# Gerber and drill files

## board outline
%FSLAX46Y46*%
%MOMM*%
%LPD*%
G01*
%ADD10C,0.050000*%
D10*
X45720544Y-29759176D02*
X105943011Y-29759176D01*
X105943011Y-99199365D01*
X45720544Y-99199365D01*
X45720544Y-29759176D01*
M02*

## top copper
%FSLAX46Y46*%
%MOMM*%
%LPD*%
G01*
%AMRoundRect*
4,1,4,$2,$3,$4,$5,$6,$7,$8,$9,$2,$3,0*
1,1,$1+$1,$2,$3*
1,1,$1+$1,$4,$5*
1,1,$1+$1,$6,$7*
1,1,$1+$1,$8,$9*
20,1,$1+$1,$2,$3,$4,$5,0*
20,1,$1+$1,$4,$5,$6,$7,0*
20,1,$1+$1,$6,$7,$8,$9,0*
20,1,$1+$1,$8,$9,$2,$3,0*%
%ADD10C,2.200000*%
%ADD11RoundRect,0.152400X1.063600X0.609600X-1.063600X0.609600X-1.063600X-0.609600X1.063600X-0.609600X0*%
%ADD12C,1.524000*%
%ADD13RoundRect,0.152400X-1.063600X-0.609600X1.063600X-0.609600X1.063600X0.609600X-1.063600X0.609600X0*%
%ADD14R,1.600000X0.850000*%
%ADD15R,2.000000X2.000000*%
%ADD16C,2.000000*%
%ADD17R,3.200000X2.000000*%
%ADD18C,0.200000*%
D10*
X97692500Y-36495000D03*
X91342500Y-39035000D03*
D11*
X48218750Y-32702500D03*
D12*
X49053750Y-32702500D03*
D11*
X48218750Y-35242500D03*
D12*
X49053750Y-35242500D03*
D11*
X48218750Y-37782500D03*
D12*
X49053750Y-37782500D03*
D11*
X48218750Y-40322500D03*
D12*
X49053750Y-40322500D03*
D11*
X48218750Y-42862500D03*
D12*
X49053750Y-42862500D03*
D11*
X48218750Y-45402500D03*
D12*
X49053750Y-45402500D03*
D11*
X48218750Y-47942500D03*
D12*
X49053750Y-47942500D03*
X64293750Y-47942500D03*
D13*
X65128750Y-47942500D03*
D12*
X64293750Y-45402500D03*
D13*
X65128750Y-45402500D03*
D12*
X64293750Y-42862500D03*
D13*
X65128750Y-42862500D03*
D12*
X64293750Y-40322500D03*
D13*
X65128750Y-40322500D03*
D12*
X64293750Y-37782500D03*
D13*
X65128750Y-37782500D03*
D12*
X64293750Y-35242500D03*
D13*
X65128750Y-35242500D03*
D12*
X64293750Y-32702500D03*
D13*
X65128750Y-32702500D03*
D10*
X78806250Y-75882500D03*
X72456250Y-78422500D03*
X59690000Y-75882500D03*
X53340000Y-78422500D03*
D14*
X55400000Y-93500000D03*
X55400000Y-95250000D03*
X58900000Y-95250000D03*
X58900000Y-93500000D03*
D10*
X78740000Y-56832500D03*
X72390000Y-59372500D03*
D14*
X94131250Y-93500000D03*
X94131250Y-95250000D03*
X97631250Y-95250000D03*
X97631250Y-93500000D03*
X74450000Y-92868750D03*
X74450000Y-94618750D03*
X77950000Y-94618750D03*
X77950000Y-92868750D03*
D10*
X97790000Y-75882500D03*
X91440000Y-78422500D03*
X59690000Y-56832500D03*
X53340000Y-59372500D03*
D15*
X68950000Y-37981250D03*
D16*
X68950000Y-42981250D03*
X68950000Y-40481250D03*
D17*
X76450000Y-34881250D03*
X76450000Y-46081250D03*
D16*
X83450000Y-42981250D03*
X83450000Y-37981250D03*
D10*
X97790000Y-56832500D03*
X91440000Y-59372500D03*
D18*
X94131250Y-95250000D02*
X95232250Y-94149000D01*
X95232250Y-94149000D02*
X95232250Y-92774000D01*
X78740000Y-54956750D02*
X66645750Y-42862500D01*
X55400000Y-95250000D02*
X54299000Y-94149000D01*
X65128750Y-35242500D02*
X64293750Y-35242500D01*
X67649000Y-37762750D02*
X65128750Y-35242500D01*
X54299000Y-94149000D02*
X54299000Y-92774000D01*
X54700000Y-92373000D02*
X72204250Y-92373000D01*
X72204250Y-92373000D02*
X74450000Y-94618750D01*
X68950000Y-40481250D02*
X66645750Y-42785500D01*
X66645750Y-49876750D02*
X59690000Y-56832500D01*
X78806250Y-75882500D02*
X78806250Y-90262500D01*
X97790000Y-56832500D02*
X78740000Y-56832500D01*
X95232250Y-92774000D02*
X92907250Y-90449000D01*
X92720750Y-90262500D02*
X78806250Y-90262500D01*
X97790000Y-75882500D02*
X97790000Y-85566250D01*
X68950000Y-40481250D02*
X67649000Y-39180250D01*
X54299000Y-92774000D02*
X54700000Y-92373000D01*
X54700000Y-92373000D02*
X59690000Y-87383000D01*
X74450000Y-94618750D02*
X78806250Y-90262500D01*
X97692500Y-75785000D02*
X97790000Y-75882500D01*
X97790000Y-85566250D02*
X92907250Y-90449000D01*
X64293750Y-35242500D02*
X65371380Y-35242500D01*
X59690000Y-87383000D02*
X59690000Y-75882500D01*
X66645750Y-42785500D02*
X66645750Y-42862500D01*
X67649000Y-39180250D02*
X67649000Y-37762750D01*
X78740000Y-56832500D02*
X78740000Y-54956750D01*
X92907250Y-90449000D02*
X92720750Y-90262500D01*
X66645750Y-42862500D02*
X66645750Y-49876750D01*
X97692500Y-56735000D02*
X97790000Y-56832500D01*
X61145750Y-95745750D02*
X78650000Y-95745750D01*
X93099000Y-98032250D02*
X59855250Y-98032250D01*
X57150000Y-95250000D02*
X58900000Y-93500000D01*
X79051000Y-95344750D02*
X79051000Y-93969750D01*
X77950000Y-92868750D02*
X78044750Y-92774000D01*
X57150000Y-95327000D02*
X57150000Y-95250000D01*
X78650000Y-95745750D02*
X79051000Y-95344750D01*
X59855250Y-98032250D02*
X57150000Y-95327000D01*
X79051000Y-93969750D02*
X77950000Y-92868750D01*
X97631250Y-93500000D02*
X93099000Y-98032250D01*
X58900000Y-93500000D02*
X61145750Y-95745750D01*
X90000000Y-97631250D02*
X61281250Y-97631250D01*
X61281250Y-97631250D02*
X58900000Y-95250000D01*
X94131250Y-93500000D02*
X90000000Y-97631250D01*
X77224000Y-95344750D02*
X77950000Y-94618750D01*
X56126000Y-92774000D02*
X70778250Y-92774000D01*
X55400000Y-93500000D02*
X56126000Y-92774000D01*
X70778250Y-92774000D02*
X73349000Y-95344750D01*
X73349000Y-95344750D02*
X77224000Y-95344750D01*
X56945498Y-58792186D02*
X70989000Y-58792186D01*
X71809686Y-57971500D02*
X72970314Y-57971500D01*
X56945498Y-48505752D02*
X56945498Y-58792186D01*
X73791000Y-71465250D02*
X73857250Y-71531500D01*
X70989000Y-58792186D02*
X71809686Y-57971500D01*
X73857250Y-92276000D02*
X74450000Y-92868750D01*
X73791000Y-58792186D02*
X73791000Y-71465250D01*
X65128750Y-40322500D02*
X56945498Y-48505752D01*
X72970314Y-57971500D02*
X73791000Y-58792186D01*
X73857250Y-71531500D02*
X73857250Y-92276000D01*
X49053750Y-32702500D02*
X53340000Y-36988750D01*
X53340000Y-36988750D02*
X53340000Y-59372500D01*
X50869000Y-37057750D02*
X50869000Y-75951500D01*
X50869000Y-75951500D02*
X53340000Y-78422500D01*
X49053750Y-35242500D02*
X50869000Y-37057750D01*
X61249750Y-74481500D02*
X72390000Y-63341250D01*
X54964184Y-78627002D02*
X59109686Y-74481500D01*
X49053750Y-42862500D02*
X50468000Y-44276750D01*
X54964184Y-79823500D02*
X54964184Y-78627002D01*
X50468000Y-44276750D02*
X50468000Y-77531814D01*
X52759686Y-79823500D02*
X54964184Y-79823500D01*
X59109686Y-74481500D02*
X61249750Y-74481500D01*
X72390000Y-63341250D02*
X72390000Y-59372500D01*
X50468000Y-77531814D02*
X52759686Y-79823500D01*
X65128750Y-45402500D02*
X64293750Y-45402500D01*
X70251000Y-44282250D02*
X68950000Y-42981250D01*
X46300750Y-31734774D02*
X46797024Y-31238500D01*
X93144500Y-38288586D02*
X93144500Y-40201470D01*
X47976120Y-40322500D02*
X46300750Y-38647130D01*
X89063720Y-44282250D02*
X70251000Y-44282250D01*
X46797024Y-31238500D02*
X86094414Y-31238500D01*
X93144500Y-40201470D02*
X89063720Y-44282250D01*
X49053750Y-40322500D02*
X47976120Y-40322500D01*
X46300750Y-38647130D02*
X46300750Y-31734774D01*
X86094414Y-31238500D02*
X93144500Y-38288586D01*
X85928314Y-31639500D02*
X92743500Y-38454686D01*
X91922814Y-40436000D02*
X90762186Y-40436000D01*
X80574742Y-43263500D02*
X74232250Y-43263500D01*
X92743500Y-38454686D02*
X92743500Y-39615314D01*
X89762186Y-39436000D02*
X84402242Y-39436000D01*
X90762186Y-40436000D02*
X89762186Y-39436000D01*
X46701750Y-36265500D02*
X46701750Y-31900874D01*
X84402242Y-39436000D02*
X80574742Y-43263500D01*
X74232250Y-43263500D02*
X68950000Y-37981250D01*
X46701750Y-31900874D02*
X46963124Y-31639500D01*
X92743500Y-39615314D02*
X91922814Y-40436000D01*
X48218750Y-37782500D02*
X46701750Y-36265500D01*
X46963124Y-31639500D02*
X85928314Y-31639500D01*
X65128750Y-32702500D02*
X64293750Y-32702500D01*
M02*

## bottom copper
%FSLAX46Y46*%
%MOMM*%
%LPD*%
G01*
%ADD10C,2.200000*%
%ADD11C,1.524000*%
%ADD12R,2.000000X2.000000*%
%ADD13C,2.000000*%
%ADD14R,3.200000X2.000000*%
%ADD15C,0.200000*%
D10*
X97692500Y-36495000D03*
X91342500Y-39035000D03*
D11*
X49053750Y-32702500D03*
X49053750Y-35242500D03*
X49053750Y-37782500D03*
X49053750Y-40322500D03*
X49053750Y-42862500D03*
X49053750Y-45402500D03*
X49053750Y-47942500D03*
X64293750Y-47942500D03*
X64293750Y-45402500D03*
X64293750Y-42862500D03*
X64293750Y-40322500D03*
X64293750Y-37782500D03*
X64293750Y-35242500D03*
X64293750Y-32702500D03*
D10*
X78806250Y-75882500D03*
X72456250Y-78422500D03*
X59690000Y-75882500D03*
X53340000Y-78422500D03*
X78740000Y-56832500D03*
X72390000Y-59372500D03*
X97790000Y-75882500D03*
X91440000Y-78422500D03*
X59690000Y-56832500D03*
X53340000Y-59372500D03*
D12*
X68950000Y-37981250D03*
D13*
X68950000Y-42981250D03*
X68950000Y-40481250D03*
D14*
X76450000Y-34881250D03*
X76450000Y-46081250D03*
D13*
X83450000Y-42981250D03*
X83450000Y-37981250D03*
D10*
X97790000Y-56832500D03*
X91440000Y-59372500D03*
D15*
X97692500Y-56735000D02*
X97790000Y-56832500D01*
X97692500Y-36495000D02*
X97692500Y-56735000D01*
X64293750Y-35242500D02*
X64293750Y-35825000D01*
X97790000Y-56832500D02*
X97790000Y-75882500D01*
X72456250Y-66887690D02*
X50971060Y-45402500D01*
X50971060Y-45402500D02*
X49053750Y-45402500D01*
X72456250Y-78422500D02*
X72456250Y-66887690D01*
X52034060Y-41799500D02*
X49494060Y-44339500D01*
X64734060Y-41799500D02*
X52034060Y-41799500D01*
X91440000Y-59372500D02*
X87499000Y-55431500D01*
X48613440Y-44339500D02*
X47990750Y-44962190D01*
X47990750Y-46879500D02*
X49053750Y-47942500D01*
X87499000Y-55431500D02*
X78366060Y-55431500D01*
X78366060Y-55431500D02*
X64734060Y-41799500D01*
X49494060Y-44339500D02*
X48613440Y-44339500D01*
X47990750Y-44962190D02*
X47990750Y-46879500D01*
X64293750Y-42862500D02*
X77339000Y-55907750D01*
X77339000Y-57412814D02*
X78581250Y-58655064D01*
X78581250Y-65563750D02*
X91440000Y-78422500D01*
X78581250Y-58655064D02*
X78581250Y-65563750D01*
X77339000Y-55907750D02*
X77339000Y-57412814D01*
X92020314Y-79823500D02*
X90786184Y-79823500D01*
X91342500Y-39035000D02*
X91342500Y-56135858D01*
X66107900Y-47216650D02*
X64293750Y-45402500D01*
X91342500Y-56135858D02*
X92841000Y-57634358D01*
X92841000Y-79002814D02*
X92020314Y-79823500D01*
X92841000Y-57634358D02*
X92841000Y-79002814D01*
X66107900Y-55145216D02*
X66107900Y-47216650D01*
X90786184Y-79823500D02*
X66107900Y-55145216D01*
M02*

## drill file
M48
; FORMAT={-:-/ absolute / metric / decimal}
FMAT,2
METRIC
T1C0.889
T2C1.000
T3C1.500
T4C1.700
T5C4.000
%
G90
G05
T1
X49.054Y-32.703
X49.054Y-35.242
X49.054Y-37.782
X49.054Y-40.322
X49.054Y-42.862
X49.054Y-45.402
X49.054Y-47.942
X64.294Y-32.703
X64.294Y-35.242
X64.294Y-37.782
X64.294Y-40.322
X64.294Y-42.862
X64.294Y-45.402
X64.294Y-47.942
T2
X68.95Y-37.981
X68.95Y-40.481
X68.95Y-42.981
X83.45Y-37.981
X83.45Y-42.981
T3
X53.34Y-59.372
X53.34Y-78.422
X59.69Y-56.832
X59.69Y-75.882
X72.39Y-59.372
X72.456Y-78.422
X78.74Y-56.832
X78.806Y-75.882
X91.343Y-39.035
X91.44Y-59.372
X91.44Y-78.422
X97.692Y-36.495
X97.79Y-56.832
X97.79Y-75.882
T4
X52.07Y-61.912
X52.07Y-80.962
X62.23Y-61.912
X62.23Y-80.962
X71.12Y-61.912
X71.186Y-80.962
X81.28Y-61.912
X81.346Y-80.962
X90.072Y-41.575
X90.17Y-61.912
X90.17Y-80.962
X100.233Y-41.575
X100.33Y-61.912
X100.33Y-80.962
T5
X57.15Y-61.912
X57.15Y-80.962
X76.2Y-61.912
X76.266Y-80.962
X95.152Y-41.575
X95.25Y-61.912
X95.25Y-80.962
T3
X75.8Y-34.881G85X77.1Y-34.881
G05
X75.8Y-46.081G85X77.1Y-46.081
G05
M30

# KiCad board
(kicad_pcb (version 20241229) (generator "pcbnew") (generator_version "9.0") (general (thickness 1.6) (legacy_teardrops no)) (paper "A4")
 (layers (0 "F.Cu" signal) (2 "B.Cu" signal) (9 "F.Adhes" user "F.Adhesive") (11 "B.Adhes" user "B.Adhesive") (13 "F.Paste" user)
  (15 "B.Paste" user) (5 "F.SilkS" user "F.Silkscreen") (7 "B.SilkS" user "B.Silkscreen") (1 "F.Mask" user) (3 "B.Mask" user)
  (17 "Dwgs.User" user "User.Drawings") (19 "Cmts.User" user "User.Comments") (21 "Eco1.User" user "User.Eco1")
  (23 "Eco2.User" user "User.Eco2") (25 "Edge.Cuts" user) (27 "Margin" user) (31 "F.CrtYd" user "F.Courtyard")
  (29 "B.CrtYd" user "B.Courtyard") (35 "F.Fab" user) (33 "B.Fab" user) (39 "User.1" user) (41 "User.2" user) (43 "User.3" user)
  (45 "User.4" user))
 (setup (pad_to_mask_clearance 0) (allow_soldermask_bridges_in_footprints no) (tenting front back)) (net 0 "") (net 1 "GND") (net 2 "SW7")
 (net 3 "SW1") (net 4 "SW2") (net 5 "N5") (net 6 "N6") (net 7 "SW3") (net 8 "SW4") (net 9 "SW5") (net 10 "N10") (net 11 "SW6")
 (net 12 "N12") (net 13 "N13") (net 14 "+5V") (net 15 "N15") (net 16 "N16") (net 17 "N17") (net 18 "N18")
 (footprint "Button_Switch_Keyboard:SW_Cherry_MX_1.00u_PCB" (layer "F.Cu") (at 97.6925 36.495)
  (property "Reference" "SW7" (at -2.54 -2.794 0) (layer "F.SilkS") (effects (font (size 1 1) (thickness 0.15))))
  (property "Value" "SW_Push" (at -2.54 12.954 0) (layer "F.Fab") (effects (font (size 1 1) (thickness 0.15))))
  (pad "" np_thru_hole circle (at -7.62 5.08) (size 1.7 1.7) (drill 1.7) (layers "*.Cu" "*.Mask"))
  (pad "" np_thru_hole circle (at -2.54 5.08) (size 4 4) (drill 4) (layers "*.Cu" "*.Mask"))
  (pad "" np_thru_hole circle (at 2.54 5.08) (size 1.7 1.7) (drill 1.7) (layers "*.Cu" "*.Mask"))
  (pad "1" thru_hole circle (at 0 0) (size 2.2 2.2) (drill 1.5) (layers "*.Cu" "*.Mask") (remove_unused_layers no) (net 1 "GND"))
  (pad "2" thru_hole circle (at -6.35 2.54) (size 2.2 2.2) (drill 1.5) (layers "*.Cu" "*.Mask") (remove_unused_layers no) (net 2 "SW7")))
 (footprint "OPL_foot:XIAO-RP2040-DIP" (layer "F.Cu") (at 56.67375 40.3225)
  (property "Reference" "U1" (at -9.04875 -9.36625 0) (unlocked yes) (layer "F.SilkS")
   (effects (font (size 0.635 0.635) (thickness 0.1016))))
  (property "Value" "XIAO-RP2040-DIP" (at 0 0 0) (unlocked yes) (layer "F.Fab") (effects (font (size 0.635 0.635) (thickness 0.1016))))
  (pad "1" smd roundrect (at -8.455 -7.62 180) (size 2.432 1.524) (layers "F.Cu" "F.Mask") (roundrect_rratio 0.1) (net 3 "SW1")
   (thermal_bridge_angle 45))
  (pad "1" thru_hole circle (at -7.62 -7.62 180) (size 1.524 1.524) (drill 0.889) (layers "*.Cu" "*.Mask") (remove_unused_layers no)
   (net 3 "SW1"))
  (pad "2" smd roundrect (at -8.455 -5.08 180) (size 2.432 1.524) (layers "F.Cu" "F.Mask") (roundrect_rratio 0.1) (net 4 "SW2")
   (thermal_bridge_angle 45))
  (pad "2" thru_hole circle (at -7.62 -5.08 180) (size 1.524 1.524) (drill 0.889) (layers "*.Cu" "*.Mask") (remove_unused_layers no)
   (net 4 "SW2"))
  (pad "3" smd roundrect (at -8.455 -2.54 180) (size 2.432 1.524) (layers "F.Cu" "F.Mask") (roundrect_rratio 0.1) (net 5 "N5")
   (thermal_bridge_angle 45))
  (pad "3" thru_hole circle (at -7.62 -2.54 180) (size 1.524 1.524) (drill 0.889) (layers "*.Cu" "*.Mask") (remove_unused_layers no)
   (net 5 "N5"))
  (pad "4" smd roundrect (at -8.455 0 180) (size 2.432 1.524) (layers "F.Cu" "F.Mask") (roundrect_rratio 0.1) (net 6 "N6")
   (thermal_bridge_angle 45))
  (pad "4" thru_hole circle (at -7.62 0 180) (size 1.524 1.524) (drill 0.889) (layers "*.Cu" "*.Mask") (remove_unused_layers no)
   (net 6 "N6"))
  (pad "5" smd roundrect (at -8.455 2.54 180) (size 2.432 1.524) (layers "F.Cu" "F.Mask") (roundrect_rratio 0.1) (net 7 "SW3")
   (thermal_bridge_angle 45))
  (pad "5" thru_hole circle (at -7.62 2.54 180) (size 1.524 1.524) (drill 0.889) (layers "*.Cu" "*.Mask") (remove_unused_layers no)
   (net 7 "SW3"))
  (pad "6" smd roundrect (at -8.455 5.08 180) (size 2.432 1.524) (layers "F.Cu" "F.Mask") (roundrect_rratio 0.1) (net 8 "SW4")
   (thermal_bridge_angle 45))
  (pad "6" thru_hole circle (at -7.62 5.08 180) (size 1.524 1.524) (drill 0.889) (layers "*.Cu" "*.Mask") (remove_unused_layers no)
   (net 8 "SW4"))
  (pad "7" smd roundrect (at -8.455 7.62 180) (size 2.432 1.524) (layers "F.Cu" "F.Mask") (roundrect_rratio 0.1) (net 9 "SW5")
   (thermal_bridge_angle 45))
  (pad "7" thru_hole circle (at -7.62 7.62 180) (size 1.524 1.524) (drill 0.889) (layers "*.Cu" "*.Mask") (remove_unused_layers no)
   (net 9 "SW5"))
  (pad "8" thru_hole circle (at 7.62 7.62) (size 1.524 1.524) (drill 0.889) (layers "*.Cu" "*.Mask") (remove_unused_layers no)
   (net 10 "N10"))
  (pad "8" smd roundrect (at 8.455 7.62) (size 2.432 1.524) (layers "F.Cu" "F.Mask") (roundrect_rratio 0.1) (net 10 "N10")
   (thermal_bridge_angle 45))
  (pad "9" thru_hole circle (at 7.62 5.08) (size 1.524 1.524) (drill 0.889) (layers "*.Cu" "*.Mask") (remove_unused_layers no) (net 2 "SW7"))
  (pad "9" smd roundrect (at 8.455 5.08) (size 2.432 1.524) (layers "F.Cu" "F.Mask") (roundrect_rratio 0.1) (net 2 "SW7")
   (thermal_bridge_angle 45))
  (pad "10" thru_hole circle (at 7.62 2.54) (size 1.524 1.524) (drill 0.889) (layers "*.Cu" "*.Mask") (remove_unused_layers no)
   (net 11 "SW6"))
  (pad "10" smd roundrect (at 8.455 2.54) (size 2.432 1.524) (layers "F.Cu" "F.Mask") (roundrect_rratio 0.1) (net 11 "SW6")
   (thermal_bridge_angle 45))
  (pad "11" thru_hole circle (at 7.62 0) (size 1.524 1.524) (drill 0.889) (layers "*.Cu" "*.Mask") (remove_unused_layers no) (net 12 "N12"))
  (pad "11" smd roundrect (at 8.455 0) (size 2.432 1.524) (layers "F.Cu" "F.Mask") (roundrect_rratio 0.1) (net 12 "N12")
   (thermal_bridge_angle 45))
  (pad "12" thru_hole circle (at 7.62 -2.54) (size 1.524 1.524) (drill 0.889) (layers "*.Cu" "*.Mask") (remove_unused_layers no)
   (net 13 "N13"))
  (pad "12" smd roundrect (at 8.455 -2.54) (size 2.432 1.524) (layers "F.Cu" "F.Mask") (roundrect_rratio 0.1) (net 13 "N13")
   (thermal_bridge_angle 45))
  (pad "13" thru_hole circle (at 7.62 -5.08) (size 1.524 1.524) (drill 0.889) (layers "*.Cu" "*.Mask") (remove_unused_layers no)
   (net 1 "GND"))
  (pad "13" smd roundrect (at 8.455 -5.08) (size 2.432 1.524) (layers "F.Cu" "F.Mask") (roundrect_rratio 0.1) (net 1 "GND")
   (thermal_bridge_angle 45))
  (pad "14" thru_hole circle (at 7.62 -7.62) (size 1.524 1.524) (drill 0.889) (layers "*.Cu" "*.Mask") (remove_unused_layers no)
   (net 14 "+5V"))
  (pad "14" smd roundrect (at 8.455 -7.62) (size 2.432 1.524) (layers "F.Cu" "F.Mask") (roundrect_rratio 0.1) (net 14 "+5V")
   (thermal_bridge_angle 45)))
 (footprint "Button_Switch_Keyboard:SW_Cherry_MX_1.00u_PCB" (layer "F.Cu") (at 78.80625 75.8825)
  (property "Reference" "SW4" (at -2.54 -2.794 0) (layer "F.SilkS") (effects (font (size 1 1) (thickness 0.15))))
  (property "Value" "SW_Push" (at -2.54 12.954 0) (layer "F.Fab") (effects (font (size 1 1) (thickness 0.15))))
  (pad "" np_thru_hole circle (at -7.62 5.08) (size 1.7 1.7) (drill 1.7) (layers "*.Cu" "*.Mask"))
  (pad "" np_thru_hole circle (at -2.54 5.08) (size 4 4) (drill 4) (layers "*.Cu" "*.Mask"))
  (pad "" np_thru_hole circle (at 2.54 5.08) (size 1.7 1.7) (drill 1.7) (layers "*.Cu" "*.Mask"))
  (pad "1" thru_hole circle (at 0 0) (size 2.2 2.2) (drill 1.5) (layers "*.Cu" "*.Mask") (remove_unused_layers no) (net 1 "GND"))
  (pad "2" thru_hole circle (at -6.35 2.54) (size 2.2 2.2) (drill 1.5) (layers "*.Cu" "*.Mask") (remove_unused_layers no) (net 8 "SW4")))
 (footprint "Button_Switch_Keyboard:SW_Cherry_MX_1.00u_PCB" (layer "F.Cu") (at 59.69 75.8825)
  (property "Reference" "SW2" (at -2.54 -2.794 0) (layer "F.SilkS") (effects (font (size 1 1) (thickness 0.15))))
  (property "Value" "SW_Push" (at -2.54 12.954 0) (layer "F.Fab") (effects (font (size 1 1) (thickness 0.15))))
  (pad "" np_thru_hole circle (at -7.62 5.08) (size 1.7 1.7) (drill 1.7) (layers "*.Cu" "*.Mask"))
  (pad "" np_thru_hole circle (at -2.54 5.08) (size 4 4) (drill 4) (layers "*.Cu" "*.Mask"))
  (pad "" np_thru_hole circle (at 2.54 5.08) (size 1.7 1.7) (drill 1.7) (layers "*.Cu" "*.Mask"))
  (pad "1" thru_hole circle (at 0 0) (size 2.2 2.2) (drill 1.5) (layers "*.Cu" "*.Mask") (remove_unused_layers no) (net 1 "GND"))
  (pad "2" thru_hole circle (at -6.35 2.54) (size 2.2 2.2) (drill 1.5) (layers "*.Cu" "*.Mask") (remove_unused_layers no) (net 4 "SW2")))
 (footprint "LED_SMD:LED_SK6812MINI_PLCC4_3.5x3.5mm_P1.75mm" (layer "F.Cu") (at 57.15 94.375)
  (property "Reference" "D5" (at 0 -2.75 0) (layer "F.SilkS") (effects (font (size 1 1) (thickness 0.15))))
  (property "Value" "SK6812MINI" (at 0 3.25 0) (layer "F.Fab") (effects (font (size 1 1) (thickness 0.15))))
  (pad "1" smd rect (at -1.75 -0.875) (size 1.6 0.85) (layers "F.Cu" "F.Mask" "F.Paste") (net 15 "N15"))
  (pad "2" smd rect (at -1.75 0.875) (size 1.6 0.85) (layers "F.Cu" "F.Mask" "F.Paste") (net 1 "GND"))
  (pad "3" smd rect (at 1.75 0.875) (size 1.6 0.85) (layers "F.Cu" "F.Mask" "F.Paste") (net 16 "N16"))
  (pad "4" smd rect (at 1.75 -0.875) (size 1.6 0.85) (layers "F.Cu" "F.Mask" "F.Paste") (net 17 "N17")))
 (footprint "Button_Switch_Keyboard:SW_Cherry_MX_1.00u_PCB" (layer "F.Cu") (at 78.74 56.8325)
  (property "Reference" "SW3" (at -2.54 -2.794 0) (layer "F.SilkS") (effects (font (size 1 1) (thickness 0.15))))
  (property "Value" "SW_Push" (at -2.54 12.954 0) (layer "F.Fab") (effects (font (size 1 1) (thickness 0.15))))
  (pad "" np_thru_hole circle (at -7.62 5.08) (size 1.7 1.7) (drill 1.7) (layers "*.Cu" "*.Mask"))
  (pad "" np_thru_hole circle (at -2.54 5.08) (size 4 4) (drill 4) (layers "*.Cu" "*.Mask"))
  (pad "" np_thru_hole circle (at 2.54 5.08) (size 1.7 1.7) (drill 1.7) (layers "*.Cu" "*.Mask"))
  (pad "1" thru_hole circle (at 0 0) (size 2.2 2.2) (drill 1.5) (layers "*.Cu" "*.Mask") (remove_unused_layers no) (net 1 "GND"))
  (pad "2" thru_hole circle (at -6.35 2.54) (size 2.2 2.2) (drill 1.5) (layers "*.Cu" "*.Mask") (remove_unused_layers no) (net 7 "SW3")))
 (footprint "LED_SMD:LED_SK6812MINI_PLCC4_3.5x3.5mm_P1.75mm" (layer "F.Cu") (at 95.88125 94.375)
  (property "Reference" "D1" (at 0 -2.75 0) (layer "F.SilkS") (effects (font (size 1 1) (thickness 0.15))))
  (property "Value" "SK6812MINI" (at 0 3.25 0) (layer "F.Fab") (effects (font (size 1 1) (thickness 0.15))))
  (pad "1" smd rect (at -1.75 -0.875) (size 1.6 0.85) (layers "F.Cu" "F.Mask" "F.Paste") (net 16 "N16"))
  (pad "2" smd rect (at -1.75 0.875) (size 1.6 0.85) (layers "F.Cu" "F.Mask" "F.Paste") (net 1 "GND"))
  (pad "3" smd rect (at 1.75 0.875) (size 1.6 0.85) (layers "F.Cu" "F.Mask" "F.Paste") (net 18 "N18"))
  (pad "4" smd rect (at 1.75 -0.875) (size 1.6 0.85) (layers "F.Cu" "F.Mask" "F.Paste") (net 17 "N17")))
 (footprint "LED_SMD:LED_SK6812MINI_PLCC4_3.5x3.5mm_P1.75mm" (layer "F.Cu") (at 76.2 93.74375)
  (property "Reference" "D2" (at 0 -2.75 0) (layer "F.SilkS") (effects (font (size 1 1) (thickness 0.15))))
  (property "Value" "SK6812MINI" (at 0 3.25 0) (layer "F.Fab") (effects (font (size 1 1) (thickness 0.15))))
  (pad "1" smd rect (at -1.75 -0.875) (size 1.6 0.85) (layers "F.Cu" "F.Mask" "F.Paste") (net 12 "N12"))
  (pad "2" smd rect (at -1.75 0.875) (size 1.6 0.85) (layers "F.Cu" "F.Mask" "F.Paste") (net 1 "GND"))
  (pad "3" smd rect (at 1.75 0.875) (size 1.6 0.85) (layers "F.Cu" "F.Mask" "F.Paste") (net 15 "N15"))
  (pad "4" smd rect (at 1.75 -0.875) (size 1.6 0.85) (layers "F.Cu" "F.Mask" "F.Paste") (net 17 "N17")))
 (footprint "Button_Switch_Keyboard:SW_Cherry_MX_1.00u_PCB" (layer "F.Cu") (at 97.79 75.8825)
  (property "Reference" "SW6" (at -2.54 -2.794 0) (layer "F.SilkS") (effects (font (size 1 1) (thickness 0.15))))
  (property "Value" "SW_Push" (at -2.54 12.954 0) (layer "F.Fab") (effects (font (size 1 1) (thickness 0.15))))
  (pad "" np_thru_hole circle (at -7.62 5.08) (size 1.7 1.7) (drill 1.7) (layers "*.Cu" "*.Mask"))
  (pad "" np_thru_hole circle (at -2.54 5.08) (size 4 4) (drill 4) (layers "*.Cu" "*.Mask"))
  (pad "" np_thru_hole circle (at 2.54 5.08) (size 1.7 1.7) (drill 1.7) (layers "*.Cu" "*.Mask"))
  (pad "1" thru_hole circle (at 0 0) (size 2.2 2.2) (drill 1.5) (layers "*.Cu" "*.Mask") (remove_unused_layers no) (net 1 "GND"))
  (pad "2" thru_hole circle (at -6.35 2.54) (size 2.2 2.2) (drill 1.5) (layers "*.Cu" "*.Mask") (remove_unused_layers no) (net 11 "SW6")))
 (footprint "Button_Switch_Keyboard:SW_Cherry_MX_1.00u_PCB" (layer "F.Cu") (at 59.69 56.8325)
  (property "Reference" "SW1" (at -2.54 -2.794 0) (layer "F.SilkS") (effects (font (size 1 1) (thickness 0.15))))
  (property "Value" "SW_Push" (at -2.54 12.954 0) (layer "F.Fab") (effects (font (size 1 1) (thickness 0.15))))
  (pad "" np_thru_hole circle (at -7.62 5.08) (size 1.7 1.7) (drill 1.7) (layers "*.Cu" "*.Mask"))
  (pad "" np_thru_hole circle (at -2.54 5.08) (size 4 4) (drill 4) (layers "*.Cu" "*.Mask"))
  (pad "" np_thru_hole circle (at 2.54 5.08) (size 1.7 1.7) (drill 1.7) (layers "*.Cu" "*.Mask"))
  (pad "1" thru_hole circle (at 0 0) (size 2.2 2.2) (drill 1.5) (layers "*.Cu" "*.Mask") (remove_unused_layers no) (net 1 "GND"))
  (pad "2" thru_hole circle (at -6.35 2.54) (size 2.2 2.2) (drill 1.5) (layers "*.Cu" "*.Mask") (remove_unused_layers no) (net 3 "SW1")))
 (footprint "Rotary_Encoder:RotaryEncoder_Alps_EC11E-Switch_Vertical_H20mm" (layer "F.Cu") (at 68.95 37.98125)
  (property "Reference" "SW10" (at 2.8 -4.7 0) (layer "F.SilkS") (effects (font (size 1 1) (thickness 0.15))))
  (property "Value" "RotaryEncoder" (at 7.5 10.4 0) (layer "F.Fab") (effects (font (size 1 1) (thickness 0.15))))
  (pad "A" thru_hole rect (at 0 0) (size 2 2) (drill 1) (layers "*.Cu" "*.Mask") (remove_unused_layers no) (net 5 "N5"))
  (pad "B" thru_hole circle (at 0 5) (size 2 2) (drill 1) (layers "*.Cu" "*.Mask") (remove_unused_layers no) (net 6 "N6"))
  (pad "C" thru_hole circle (at 0 2.5) (size 2 2) (drill 1) (layers "*.Cu" "*.Mask") (remove_unused_layers no) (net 1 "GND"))
  (pad "MP" thru_hole rect (at 7.5 -3.1) (size 3.2 2) (drill oval 2.8 1.5) (layers "*.Cu" "*.Mask") (remove_unused_layers no))
  (pad "MP" thru_hole rect (at 7.5 8.1) (size 3.2 2) (drill oval 2.8 1.5) (layers "*.Cu" "*.Mask") (remove_unused_layers no))
  (pad "S1" thru_hole circle (at 14.5 5) (size 2 2) (drill 1) (layers "*.Cu" "*.Mask") (remove_unused_layers no))
  (pad "S2" thru_hole circle (at 14.5 0) (size 2 2) (drill 1) (layers "*.Cu" "*.Mask") (remove_unused_layers no)))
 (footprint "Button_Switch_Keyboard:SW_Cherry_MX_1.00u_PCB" (layer "F.Cu") (at 97.79 56.8325)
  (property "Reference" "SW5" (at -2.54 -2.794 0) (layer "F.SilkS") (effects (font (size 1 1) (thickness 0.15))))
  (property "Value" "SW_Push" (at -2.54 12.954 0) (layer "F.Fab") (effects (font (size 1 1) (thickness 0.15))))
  (pad "" np_thru_hole circle (at -7.62 5.08) (size 1.7 1.7) (drill 1.7) (layers "*.Cu" "*.Mask"))
  (pad "" np_thru_hole circle (at -2.54 5.08) (size 4 4) (drill 4) (layers "*.Cu" "*.Mask"))
  (pad "" np_thru_hole circle (at 2.54 5.08) (size 1.7 1.7) (drill 1.7) (layers "*.Cu" "*.Mask"))
  (pad "1" thru_hole circle (at 0 0) (size 2.2 2.2) (drill 1.5) (layers "*.Cu" "*.Mask") (remove_unused_layers no) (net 1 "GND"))
  (pad "2" thru_hole circle (at -6.35 2.54) (size 2.2 2.2) (drill 1.5) (layers "*.Cu" "*.Mask") (remove_unused_layers no) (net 9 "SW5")))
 (gr_rect (start 45.720544 29.759176) (end 105.943011 99.199365) (stroke (width 0.05) (type default)) (fill no) (layer "Edge.Cuts"))
 (segment (start 94.13125 95.25) (end 95.23225 94.149) (width 0.2) (layer "F.Cu") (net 1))
 (segment (start 95.23225 94.149) (end 95.23225 92.774) (width 0.2) (layer "F.Cu") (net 1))
 (segment (start 78.74 54.95675) (end 66.64575 42.8625) (width 0.2) (layer "F.Cu") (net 1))
 (segment (start 55.4 95.25) (end 54.299 94.149) (width 0.2) (layer "F.Cu") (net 1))
 (segment (start 65.12875 35.2425) (end 64.29375 35.2425) (width 0.2) (layer "F.Cu") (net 1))
 (segment (start 67.649 37.76275) (end 65.12875 35.2425) (width 0.2) (layer "F.Cu") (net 1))
 (segment (start 54.299 94.149) (end 54.299 92.774) (width 0.2) (layer "F.Cu") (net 1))
 (segment (start 54.7 92.373) (end 72.20425 92.373) (width 0.2) (layer "F.Cu") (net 1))
 (segment (start 72.20425 92.373) (end 74.45 94.61875) (width 0.2) (layer "F.Cu") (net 1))
 (segment (start 68.95 40.48125) (end 66.64575 42.7855) (width 0.2) (layer "F.Cu") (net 1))
 (segment (start 66.64575 49.87675) (end 59.69 56.8325) (width 0.2) (layer "F.Cu") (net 1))
 (segment (start 78.80625 75.8825) (end 78.80625 90.2625) (width 0.2) (layer "F.Cu") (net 1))
 (segment (start 97.79 56.8325) (end 78.74 56.8325) (width 0.2) (layer "F.Cu") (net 1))
 (segment (start 95.23225 92.774) (end 92.90725 90.449) (width 0.2) (layer "F.Cu") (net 1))
 (segment (start 92.72075 90.2625) (end 78.80625 90.2625) (width 0.2) (layer "F.Cu") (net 1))
 (segment (start 97.79 75.8825) (end 97.79 85.56625) (width 0.2) (layer "F.Cu") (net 1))
 (segment (start 68.95 40.48125) (end 67.649 39.18025) (width 0.2) (layer "F.Cu") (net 1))
 (segment (start 54.299 92.774) (end 54.7 92.373) (width 0.2) (layer "F.Cu") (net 1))
 (segment (start 54.7 92.373) (end 59.69 87.383) (width 0.2) (layer "F.Cu") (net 1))
 (segment (start 74.45 94.61875) (end 78.80625 90.2625) (width 0.2) (layer "F.Cu") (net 1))
 (segment (start 97.6925 75.785) (end 97.79 75.8825) (width 0.2) (layer "F.Cu") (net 1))
 (segment (start 97.79 85.56625) (end 92.90725 90.449) (width 0.2) (layer "F.Cu") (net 1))
 (segment (start 64.29375 35.2425) (end 65.37138 35.2425) (width 0.2) (layer "F.Cu") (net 1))
 (segment (start 59.69 87.383) (end 59.69 75.8825) (width 0.2) (layer "F.Cu") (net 1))
 (segment (start 66.64575 42.7855) (end 66.64575 42.8625) (width 0.2) (layer "F.Cu") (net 1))
 (segment (start 67.649 39.18025) (end 67.649 37.76275) (width 0.2) (layer "F.Cu") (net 1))
 (segment (start 78.74 56.8325) (end 78.74 54.95675) (width 0.2) (layer "F.Cu") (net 1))
 (segment (start 92.90725 90.449) (end 92.72075 90.2625) (width 0.2) (layer "F.Cu") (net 1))
 (segment (start 66.64575 42.8625) (end 66.64575 49.87675) (width 0.2) (layer "F.Cu") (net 1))
 (segment (start 97.6925 56.735) (end 97.79 56.8325) (width 0.2) (layer "F.Cu") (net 1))
 (segment (start 97.6925 56.735) (end 97.79 56.8325) (width 0.2) (layer "B.Cu") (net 1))
 (segment (start 97.6925 36.495) (end 97.6925 56.735) (width 0.2) (layer "B.Cu") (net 1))
 (segment (start 64.29375 35.2425) (end 64.29375 35.825) (width 0.2) (layer "B.Cu") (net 1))
 (segment (start 97.79 56.8325) (end 97.79 75.8825) (width 0.2) (layer "B.Cu") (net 1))
 (segment (start 61.14575 95.74575) (end 78.65 95.74575) (width 0.2) (layer "F.Cu") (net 17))
 (segment (start 93.099 98.03225) (end 59.85525 98.03225) (width 0.2) (layer "F.Cu") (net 17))
 (segment (start 57.15 95.25) (end 58.9 93.5) (width 0.2) (layer "F.Cu") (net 17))
 (segment (start 79.051 95.34475) (end 79.051 93.96975) (width 0.2) (layer "F.Cu") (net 17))
 (segment (start 77.95 92.86875) (end 78.04475 92.774) (width 0.2) (layer "F.Cu") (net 17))
 (segment (start 57.15 95.327) (end 57.15 95.25) (width 0.2) (layer "F.Cu") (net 17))
 (segment (start 78.65 95.74575) (end 79.051 95.34475) (width 0.2) (layer "F.Cu") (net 17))
 (segment (start 59.85525 98.03225) (end 57.15 95.327) (width 0.2) (layer "F.Cu") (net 17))
 (segment (start 79.051 93.96975) (end 77.95 92.86875) (width 0.2) (layer "F.Cu") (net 17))
 (segment (start 97.63125 93.5) (end 93.099 98.03225) (width 0.2) (layer "F.Cu") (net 17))
 (segment (start 58.9 93.5) (end 61.14575 95.74575) (width 0.2) (layer "F.Cu") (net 17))
 (segment (start 90 97.63125) (end 61.28125 97.63125) (width 0.2) (layer "F.Cu") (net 16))
 (segment (start 61.28125 97.63125) (end 58.9 95.25) (width 0.2) (layer "F.Cu") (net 16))
 (segment (start 94.13125 93.5) (end 90 97.63125) (width 0.2) (layer "F.Cu") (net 16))
 (segment (start 77.224 95.34475) (end 77.95 94.61875) (width 0.2) (layer "F.Cu") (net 15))
 (segment (start 56.126 92.774) (end 70.77825 92.774) (width 0.2) (layer "F.Cu") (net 15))
 (segment (start 55.4 93.5) (end 56.126 92.774) (width 0.2) (layer "F.Cu") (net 15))
 (segment (start 70.77825 92.774) (end 73.349 95.34475) (width 0.2) (layer "F.Cu") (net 15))
 (segment (start 73.349 95.34475) (end 77.224 95.34475) (width 0.2) (layer "F.Cu") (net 15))
 (segment (start 56.945498 58.792186) (end 70.989 58.792186) (width 0.2) (layer "F.Cu") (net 12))
 (segment (start 71.809686 57.9715) (end 72.970314 57.9715) (width 0.2) (layer "F.Cu") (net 12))
 (segment (start 56.945498 48.505752) (end 56.945498 58.792186) (width 0.2) (layer "F.Cu") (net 12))
 (segment (start 73.791 71.46525) (end 73.85725 71.5315) (width 0.2) (layer "F.Cu") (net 12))
 (segment (start 70.989 58.792186) (end 71.809686 57.9715) (width 0.2) (layer "F.Cu") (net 12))
 (segment (start 73.85725 92.276) (end 74.45 92.86875) (width 0.2) (layer "F.Cu") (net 12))
 (segment (start 73.791 58.792186) (end 73.791 71.46525) (width 0.2) (layer "F.Cu") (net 12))
 (segment (start 65.12875 40.3225) (end 56.945498 48.505752) (width 0.2) (layer "F.Cu") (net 12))
 (segment (start 72.970314 57.9715) (end 73.791 58.792186) (width 0.2) (layer "F.Cu") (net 12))
 (segment (start 73.85725 71.5315) (end 73.85725 92.276) (width 0.2) (layer "F.Cu") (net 12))
 (segment (start 49.05375 32.7025) (end 53.34 36.98875) (width 0.2) (layer "F.Cu") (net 3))
 (segment (start 53.34 36.98875) (end 53.34 59.3725) (width 0.2) (layer "F.Cu") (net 3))
 (segment (start 50.869 37.05775) (end 50.869 75.9515) (width 0.2) (layer "F.Cu") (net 4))
 (segment (start 50.869 75.9515) (end 53.34 78.4225) (width 0.2) (layer "F.Cu") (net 4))
 (segment (start 49.05375 35.2425) (end 50.869 37.05775) (width 0.2) (layer "F.Cu") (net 4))
 (segment (start 61.24975 74.4815) (end 72.39 63.34125) (width 0.2) (layer "F.Cu") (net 7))
 (segment (start 54.964184 78.627002) (end 59.109686 74.4815) (width 0.2) (layer "F.Cu") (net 7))
 (segment (start 49.05375 42.8625) (end 50.468 44.27675) (width 0.2) (layer "F.Cu") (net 7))
 (segment (start 54.964184 79.8235) (end 54.964184 78.627002) (width 0.2) (layer "F.Cu") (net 7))
 (segment (start 50.468 44.27675) (end 50.468 77.531814) (width 0.2) (layer "F.Cu") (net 7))
 (segment (start 52.759686 79.8235) (end 54.964184 79.8235) (width 0.2) (layer "F.Cu") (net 7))
 (segment (start 59.109686 74.4815) (end 61.24975 74.4815) (width 0.2) (layer "F.Cu") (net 7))
 (segment (start 72.39 63.34125) (end 72.39 59.3725) (width 0.2) (layer "F.Cu") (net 7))
 (segment (start 50.468 77.531814) (end 52.759686 79.8235) (width 0.2) (layer "F.Cu") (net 7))
 (segment (start 72.45625 66.88769) (end 50.97106 45.4025) (width 0.2) (layer "B.Cu") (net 8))
 (segment (start 50.97106 45.4025) (end 49.05375 45.4025) (width 0.2) (layer "B.Cu") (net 8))
 (segment (start 72.45625 78.4225) (end 72.45625 66.88769) (width 0.2) (layer "B.Cu") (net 8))
 (segment (start 52.03406 41.7995) (end 49.49406 44.3395) (width 0.2) (layer "B.Cu") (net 9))
 (segment (start 64.73406 41.7995) (end 52.03406 41.7995) (width 0.2) (layer "B.Cu") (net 9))
 (segment (start 91.44 59.3725) (end 87.499 55.4315) (width 0.2) (layer "B.Cu") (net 9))
 (segment (start 48.61344 44.3395) (end 47.99075 44.96219) (width 0.2) (layer "B.Cu") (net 9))
 (segment (start 47.99075 46.8795) (end 49.05375 47.9425) (width 0.2) (layer "B.Cu") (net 9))
 (segment (start 87.499 55.4315) (end 78.36606 55.4315) (width 0.2) (layer "B.Cu") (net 9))
 (segment (start 78.36606 55.4315) (end 64.73406 41.7995) (width 0.2) (layer "B.Cu") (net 9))
 (segment (start 49.49406 44.3395) (end 48.61344 44.3395) (width 0.2) (layer "B.Cu") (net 9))
 (segment (start 47.99075 44.96219) (end 47.99075 46.8795) (width 0.2) (layer "B.Cu") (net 9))
 (segment (start 64.29375 42.8625) (end 77.339 55.90775) (width 0.2) (layer "B.Cu") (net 11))
 (segment (start 77.339 57.412814) (end 78.58125 58.655064) (width 0.2) (layer "B.Cu") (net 11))
 (segment (start 78.58125 65.56375) (end 91.44 78.4225) (width 0.2) (layer "B.Cu") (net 11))
 (segment (start 78.58125 58.655064) (end 78.58125 65.56375) (width 0.2) (layer "B.Cu") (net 11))
 (segment (start 77.339 55.90775) (end 77.339 57.412814) (width 0.2) (layer "B.Cu") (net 11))
 (segment (start 65.12875 45.4025) (end 64.29375 45.4025) (width 0.2) (layer "F.Cu") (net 2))
 (segment (start 92.020314 79.8235) (end 90.786184 79.8235) (width 0.2) (layer "B.Cu") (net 2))
 (segment (start 91.3425 39.035) (end 91.3425 56.135858) (width 0.2) (layer "B.Cu") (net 2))
 (segment (start 66.1079 47.21665) (end 64.29375 45.4025) (width 0.2) (layer "B.Cu") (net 2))
 (segment (start 91.3425 56.135858) (end 92.841 57.634358) (width 0.2) (layer "B.Cu") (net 2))
 (segment (start 92.841 79.002814) (end 92.020314 79.8235) (width 0.2) (layer "B.Cu") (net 2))
 (segment (start 92.841 57.634358) (end 92.841 79.002814) (width 0.2) (layer "B.Cu") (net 2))
 (segment (start 66.1079 55.145216) (end 66.1079 47.21665) (width 0.2) (layer "B.Cu") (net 2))
 (segment (start 90.786184 79.8235) (end 66.1079 55.145216) (width 0.2) (layer "B.Cu") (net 2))
 (segment (start 70.251 44.28225) (end 68.95 42.98125) (width 0.2) (layer "F.Cu") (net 6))
 (segment (start 46.30075 31.734774) (end 46.797024 31.2385) (width 0.2) (layer "F.Cu") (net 6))
 (segment (start 93.1445 38.288586) (end 93.1445 40.20147) (width 0.2) (layer "F.Cu") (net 6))
 (segment (start 47.97612 40.3225) (end 46.30075 38.64713) (width 0.2) (layer "F.Cu") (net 6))
 (segment (start 89.06372 44.28225) (end 70.251 44.28225) (width 0.2) (layer "F.Cu") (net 6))
 (segment (start 46.797024 31.2385) (end 86.094414 31.2385) (width 0.2) (layer "F.Cu") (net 6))
 (segment (start 93.1445 40.20147) (end 89.06372 44.28225) (width 0.2) (layer "F.Cu") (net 6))
 (segment (start 49.05375 40.3225) (end 47.97612 40.3225) (width 0.2) (layer "F.Cu") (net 6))
 (segment (start 46.30075 38.64713) (end 46.30075 31.734774) (width 0.2) (layer "F.Cu") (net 6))
 (segment (start 86.094414 31.2385) (end 93.1445 38.288586) (width 0.2) (layer "F.Cu") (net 6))
 (segment (start 85.928314 31.6395) (end 92.7435 38.454686) (width 0.2) (layer "F.Cu") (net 5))
 (segment (start 91.922814 40.436) (end 90.762186 40.436) (width 0.2) (layer "F.Cu") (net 5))
 (segment (start 80.574742 43.2635) (end 74.23225 43.2635) (width 0.2) (layer "F.Cu") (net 5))
 (segment (start 92.7435 38.454686) (end 92.7435 39.615314) (width 0.2) (layer "F.Cu") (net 5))
 (segment (start 89.762186 39.436) (end 84.402242 39.436) (width 0.2) (layer "F.Cu") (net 5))
 (segment (start 90.762186 40.436) (end 89.762186 39.436) (width 0.2) (layer "F.Cu") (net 5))
 (segment (start 46.70175 36.2655) (end 46.70175 31.900874) (width 0.2) (layer "F.Cu") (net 5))
 (segment (start 84.402242 39.436) (end 80.574742 43.2635) (width 0.2) (layer "F.Cu") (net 5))
 (segment (start 74.23225 43.2635) (end 68.95 37.98125) (width 0.2) (layer "F.Cu") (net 5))
 (segment (start 46.70175 31.900874) (end 46.963124 31.6395) (width 0.2) (layer "F.Cu") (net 5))
 (segment (start 92.7435 39.615314) (end 91.922814 40.436) (width 0.2) (layer "F.Cu") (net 5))
 (segment (start 48.21875 37.7825) (end 46.70175 36.2655) (width 0.2) (layer "F.Cu") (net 5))
 (segment (start 46.963124 31.6395) (end 85.928314 31.6395) (width 0.2) (layer "F.Cu") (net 5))
 (segment (start 65.12875 32.7025) (end 64.29375 32.7025) (width 0.2) (layer "F.Cu") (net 14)))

